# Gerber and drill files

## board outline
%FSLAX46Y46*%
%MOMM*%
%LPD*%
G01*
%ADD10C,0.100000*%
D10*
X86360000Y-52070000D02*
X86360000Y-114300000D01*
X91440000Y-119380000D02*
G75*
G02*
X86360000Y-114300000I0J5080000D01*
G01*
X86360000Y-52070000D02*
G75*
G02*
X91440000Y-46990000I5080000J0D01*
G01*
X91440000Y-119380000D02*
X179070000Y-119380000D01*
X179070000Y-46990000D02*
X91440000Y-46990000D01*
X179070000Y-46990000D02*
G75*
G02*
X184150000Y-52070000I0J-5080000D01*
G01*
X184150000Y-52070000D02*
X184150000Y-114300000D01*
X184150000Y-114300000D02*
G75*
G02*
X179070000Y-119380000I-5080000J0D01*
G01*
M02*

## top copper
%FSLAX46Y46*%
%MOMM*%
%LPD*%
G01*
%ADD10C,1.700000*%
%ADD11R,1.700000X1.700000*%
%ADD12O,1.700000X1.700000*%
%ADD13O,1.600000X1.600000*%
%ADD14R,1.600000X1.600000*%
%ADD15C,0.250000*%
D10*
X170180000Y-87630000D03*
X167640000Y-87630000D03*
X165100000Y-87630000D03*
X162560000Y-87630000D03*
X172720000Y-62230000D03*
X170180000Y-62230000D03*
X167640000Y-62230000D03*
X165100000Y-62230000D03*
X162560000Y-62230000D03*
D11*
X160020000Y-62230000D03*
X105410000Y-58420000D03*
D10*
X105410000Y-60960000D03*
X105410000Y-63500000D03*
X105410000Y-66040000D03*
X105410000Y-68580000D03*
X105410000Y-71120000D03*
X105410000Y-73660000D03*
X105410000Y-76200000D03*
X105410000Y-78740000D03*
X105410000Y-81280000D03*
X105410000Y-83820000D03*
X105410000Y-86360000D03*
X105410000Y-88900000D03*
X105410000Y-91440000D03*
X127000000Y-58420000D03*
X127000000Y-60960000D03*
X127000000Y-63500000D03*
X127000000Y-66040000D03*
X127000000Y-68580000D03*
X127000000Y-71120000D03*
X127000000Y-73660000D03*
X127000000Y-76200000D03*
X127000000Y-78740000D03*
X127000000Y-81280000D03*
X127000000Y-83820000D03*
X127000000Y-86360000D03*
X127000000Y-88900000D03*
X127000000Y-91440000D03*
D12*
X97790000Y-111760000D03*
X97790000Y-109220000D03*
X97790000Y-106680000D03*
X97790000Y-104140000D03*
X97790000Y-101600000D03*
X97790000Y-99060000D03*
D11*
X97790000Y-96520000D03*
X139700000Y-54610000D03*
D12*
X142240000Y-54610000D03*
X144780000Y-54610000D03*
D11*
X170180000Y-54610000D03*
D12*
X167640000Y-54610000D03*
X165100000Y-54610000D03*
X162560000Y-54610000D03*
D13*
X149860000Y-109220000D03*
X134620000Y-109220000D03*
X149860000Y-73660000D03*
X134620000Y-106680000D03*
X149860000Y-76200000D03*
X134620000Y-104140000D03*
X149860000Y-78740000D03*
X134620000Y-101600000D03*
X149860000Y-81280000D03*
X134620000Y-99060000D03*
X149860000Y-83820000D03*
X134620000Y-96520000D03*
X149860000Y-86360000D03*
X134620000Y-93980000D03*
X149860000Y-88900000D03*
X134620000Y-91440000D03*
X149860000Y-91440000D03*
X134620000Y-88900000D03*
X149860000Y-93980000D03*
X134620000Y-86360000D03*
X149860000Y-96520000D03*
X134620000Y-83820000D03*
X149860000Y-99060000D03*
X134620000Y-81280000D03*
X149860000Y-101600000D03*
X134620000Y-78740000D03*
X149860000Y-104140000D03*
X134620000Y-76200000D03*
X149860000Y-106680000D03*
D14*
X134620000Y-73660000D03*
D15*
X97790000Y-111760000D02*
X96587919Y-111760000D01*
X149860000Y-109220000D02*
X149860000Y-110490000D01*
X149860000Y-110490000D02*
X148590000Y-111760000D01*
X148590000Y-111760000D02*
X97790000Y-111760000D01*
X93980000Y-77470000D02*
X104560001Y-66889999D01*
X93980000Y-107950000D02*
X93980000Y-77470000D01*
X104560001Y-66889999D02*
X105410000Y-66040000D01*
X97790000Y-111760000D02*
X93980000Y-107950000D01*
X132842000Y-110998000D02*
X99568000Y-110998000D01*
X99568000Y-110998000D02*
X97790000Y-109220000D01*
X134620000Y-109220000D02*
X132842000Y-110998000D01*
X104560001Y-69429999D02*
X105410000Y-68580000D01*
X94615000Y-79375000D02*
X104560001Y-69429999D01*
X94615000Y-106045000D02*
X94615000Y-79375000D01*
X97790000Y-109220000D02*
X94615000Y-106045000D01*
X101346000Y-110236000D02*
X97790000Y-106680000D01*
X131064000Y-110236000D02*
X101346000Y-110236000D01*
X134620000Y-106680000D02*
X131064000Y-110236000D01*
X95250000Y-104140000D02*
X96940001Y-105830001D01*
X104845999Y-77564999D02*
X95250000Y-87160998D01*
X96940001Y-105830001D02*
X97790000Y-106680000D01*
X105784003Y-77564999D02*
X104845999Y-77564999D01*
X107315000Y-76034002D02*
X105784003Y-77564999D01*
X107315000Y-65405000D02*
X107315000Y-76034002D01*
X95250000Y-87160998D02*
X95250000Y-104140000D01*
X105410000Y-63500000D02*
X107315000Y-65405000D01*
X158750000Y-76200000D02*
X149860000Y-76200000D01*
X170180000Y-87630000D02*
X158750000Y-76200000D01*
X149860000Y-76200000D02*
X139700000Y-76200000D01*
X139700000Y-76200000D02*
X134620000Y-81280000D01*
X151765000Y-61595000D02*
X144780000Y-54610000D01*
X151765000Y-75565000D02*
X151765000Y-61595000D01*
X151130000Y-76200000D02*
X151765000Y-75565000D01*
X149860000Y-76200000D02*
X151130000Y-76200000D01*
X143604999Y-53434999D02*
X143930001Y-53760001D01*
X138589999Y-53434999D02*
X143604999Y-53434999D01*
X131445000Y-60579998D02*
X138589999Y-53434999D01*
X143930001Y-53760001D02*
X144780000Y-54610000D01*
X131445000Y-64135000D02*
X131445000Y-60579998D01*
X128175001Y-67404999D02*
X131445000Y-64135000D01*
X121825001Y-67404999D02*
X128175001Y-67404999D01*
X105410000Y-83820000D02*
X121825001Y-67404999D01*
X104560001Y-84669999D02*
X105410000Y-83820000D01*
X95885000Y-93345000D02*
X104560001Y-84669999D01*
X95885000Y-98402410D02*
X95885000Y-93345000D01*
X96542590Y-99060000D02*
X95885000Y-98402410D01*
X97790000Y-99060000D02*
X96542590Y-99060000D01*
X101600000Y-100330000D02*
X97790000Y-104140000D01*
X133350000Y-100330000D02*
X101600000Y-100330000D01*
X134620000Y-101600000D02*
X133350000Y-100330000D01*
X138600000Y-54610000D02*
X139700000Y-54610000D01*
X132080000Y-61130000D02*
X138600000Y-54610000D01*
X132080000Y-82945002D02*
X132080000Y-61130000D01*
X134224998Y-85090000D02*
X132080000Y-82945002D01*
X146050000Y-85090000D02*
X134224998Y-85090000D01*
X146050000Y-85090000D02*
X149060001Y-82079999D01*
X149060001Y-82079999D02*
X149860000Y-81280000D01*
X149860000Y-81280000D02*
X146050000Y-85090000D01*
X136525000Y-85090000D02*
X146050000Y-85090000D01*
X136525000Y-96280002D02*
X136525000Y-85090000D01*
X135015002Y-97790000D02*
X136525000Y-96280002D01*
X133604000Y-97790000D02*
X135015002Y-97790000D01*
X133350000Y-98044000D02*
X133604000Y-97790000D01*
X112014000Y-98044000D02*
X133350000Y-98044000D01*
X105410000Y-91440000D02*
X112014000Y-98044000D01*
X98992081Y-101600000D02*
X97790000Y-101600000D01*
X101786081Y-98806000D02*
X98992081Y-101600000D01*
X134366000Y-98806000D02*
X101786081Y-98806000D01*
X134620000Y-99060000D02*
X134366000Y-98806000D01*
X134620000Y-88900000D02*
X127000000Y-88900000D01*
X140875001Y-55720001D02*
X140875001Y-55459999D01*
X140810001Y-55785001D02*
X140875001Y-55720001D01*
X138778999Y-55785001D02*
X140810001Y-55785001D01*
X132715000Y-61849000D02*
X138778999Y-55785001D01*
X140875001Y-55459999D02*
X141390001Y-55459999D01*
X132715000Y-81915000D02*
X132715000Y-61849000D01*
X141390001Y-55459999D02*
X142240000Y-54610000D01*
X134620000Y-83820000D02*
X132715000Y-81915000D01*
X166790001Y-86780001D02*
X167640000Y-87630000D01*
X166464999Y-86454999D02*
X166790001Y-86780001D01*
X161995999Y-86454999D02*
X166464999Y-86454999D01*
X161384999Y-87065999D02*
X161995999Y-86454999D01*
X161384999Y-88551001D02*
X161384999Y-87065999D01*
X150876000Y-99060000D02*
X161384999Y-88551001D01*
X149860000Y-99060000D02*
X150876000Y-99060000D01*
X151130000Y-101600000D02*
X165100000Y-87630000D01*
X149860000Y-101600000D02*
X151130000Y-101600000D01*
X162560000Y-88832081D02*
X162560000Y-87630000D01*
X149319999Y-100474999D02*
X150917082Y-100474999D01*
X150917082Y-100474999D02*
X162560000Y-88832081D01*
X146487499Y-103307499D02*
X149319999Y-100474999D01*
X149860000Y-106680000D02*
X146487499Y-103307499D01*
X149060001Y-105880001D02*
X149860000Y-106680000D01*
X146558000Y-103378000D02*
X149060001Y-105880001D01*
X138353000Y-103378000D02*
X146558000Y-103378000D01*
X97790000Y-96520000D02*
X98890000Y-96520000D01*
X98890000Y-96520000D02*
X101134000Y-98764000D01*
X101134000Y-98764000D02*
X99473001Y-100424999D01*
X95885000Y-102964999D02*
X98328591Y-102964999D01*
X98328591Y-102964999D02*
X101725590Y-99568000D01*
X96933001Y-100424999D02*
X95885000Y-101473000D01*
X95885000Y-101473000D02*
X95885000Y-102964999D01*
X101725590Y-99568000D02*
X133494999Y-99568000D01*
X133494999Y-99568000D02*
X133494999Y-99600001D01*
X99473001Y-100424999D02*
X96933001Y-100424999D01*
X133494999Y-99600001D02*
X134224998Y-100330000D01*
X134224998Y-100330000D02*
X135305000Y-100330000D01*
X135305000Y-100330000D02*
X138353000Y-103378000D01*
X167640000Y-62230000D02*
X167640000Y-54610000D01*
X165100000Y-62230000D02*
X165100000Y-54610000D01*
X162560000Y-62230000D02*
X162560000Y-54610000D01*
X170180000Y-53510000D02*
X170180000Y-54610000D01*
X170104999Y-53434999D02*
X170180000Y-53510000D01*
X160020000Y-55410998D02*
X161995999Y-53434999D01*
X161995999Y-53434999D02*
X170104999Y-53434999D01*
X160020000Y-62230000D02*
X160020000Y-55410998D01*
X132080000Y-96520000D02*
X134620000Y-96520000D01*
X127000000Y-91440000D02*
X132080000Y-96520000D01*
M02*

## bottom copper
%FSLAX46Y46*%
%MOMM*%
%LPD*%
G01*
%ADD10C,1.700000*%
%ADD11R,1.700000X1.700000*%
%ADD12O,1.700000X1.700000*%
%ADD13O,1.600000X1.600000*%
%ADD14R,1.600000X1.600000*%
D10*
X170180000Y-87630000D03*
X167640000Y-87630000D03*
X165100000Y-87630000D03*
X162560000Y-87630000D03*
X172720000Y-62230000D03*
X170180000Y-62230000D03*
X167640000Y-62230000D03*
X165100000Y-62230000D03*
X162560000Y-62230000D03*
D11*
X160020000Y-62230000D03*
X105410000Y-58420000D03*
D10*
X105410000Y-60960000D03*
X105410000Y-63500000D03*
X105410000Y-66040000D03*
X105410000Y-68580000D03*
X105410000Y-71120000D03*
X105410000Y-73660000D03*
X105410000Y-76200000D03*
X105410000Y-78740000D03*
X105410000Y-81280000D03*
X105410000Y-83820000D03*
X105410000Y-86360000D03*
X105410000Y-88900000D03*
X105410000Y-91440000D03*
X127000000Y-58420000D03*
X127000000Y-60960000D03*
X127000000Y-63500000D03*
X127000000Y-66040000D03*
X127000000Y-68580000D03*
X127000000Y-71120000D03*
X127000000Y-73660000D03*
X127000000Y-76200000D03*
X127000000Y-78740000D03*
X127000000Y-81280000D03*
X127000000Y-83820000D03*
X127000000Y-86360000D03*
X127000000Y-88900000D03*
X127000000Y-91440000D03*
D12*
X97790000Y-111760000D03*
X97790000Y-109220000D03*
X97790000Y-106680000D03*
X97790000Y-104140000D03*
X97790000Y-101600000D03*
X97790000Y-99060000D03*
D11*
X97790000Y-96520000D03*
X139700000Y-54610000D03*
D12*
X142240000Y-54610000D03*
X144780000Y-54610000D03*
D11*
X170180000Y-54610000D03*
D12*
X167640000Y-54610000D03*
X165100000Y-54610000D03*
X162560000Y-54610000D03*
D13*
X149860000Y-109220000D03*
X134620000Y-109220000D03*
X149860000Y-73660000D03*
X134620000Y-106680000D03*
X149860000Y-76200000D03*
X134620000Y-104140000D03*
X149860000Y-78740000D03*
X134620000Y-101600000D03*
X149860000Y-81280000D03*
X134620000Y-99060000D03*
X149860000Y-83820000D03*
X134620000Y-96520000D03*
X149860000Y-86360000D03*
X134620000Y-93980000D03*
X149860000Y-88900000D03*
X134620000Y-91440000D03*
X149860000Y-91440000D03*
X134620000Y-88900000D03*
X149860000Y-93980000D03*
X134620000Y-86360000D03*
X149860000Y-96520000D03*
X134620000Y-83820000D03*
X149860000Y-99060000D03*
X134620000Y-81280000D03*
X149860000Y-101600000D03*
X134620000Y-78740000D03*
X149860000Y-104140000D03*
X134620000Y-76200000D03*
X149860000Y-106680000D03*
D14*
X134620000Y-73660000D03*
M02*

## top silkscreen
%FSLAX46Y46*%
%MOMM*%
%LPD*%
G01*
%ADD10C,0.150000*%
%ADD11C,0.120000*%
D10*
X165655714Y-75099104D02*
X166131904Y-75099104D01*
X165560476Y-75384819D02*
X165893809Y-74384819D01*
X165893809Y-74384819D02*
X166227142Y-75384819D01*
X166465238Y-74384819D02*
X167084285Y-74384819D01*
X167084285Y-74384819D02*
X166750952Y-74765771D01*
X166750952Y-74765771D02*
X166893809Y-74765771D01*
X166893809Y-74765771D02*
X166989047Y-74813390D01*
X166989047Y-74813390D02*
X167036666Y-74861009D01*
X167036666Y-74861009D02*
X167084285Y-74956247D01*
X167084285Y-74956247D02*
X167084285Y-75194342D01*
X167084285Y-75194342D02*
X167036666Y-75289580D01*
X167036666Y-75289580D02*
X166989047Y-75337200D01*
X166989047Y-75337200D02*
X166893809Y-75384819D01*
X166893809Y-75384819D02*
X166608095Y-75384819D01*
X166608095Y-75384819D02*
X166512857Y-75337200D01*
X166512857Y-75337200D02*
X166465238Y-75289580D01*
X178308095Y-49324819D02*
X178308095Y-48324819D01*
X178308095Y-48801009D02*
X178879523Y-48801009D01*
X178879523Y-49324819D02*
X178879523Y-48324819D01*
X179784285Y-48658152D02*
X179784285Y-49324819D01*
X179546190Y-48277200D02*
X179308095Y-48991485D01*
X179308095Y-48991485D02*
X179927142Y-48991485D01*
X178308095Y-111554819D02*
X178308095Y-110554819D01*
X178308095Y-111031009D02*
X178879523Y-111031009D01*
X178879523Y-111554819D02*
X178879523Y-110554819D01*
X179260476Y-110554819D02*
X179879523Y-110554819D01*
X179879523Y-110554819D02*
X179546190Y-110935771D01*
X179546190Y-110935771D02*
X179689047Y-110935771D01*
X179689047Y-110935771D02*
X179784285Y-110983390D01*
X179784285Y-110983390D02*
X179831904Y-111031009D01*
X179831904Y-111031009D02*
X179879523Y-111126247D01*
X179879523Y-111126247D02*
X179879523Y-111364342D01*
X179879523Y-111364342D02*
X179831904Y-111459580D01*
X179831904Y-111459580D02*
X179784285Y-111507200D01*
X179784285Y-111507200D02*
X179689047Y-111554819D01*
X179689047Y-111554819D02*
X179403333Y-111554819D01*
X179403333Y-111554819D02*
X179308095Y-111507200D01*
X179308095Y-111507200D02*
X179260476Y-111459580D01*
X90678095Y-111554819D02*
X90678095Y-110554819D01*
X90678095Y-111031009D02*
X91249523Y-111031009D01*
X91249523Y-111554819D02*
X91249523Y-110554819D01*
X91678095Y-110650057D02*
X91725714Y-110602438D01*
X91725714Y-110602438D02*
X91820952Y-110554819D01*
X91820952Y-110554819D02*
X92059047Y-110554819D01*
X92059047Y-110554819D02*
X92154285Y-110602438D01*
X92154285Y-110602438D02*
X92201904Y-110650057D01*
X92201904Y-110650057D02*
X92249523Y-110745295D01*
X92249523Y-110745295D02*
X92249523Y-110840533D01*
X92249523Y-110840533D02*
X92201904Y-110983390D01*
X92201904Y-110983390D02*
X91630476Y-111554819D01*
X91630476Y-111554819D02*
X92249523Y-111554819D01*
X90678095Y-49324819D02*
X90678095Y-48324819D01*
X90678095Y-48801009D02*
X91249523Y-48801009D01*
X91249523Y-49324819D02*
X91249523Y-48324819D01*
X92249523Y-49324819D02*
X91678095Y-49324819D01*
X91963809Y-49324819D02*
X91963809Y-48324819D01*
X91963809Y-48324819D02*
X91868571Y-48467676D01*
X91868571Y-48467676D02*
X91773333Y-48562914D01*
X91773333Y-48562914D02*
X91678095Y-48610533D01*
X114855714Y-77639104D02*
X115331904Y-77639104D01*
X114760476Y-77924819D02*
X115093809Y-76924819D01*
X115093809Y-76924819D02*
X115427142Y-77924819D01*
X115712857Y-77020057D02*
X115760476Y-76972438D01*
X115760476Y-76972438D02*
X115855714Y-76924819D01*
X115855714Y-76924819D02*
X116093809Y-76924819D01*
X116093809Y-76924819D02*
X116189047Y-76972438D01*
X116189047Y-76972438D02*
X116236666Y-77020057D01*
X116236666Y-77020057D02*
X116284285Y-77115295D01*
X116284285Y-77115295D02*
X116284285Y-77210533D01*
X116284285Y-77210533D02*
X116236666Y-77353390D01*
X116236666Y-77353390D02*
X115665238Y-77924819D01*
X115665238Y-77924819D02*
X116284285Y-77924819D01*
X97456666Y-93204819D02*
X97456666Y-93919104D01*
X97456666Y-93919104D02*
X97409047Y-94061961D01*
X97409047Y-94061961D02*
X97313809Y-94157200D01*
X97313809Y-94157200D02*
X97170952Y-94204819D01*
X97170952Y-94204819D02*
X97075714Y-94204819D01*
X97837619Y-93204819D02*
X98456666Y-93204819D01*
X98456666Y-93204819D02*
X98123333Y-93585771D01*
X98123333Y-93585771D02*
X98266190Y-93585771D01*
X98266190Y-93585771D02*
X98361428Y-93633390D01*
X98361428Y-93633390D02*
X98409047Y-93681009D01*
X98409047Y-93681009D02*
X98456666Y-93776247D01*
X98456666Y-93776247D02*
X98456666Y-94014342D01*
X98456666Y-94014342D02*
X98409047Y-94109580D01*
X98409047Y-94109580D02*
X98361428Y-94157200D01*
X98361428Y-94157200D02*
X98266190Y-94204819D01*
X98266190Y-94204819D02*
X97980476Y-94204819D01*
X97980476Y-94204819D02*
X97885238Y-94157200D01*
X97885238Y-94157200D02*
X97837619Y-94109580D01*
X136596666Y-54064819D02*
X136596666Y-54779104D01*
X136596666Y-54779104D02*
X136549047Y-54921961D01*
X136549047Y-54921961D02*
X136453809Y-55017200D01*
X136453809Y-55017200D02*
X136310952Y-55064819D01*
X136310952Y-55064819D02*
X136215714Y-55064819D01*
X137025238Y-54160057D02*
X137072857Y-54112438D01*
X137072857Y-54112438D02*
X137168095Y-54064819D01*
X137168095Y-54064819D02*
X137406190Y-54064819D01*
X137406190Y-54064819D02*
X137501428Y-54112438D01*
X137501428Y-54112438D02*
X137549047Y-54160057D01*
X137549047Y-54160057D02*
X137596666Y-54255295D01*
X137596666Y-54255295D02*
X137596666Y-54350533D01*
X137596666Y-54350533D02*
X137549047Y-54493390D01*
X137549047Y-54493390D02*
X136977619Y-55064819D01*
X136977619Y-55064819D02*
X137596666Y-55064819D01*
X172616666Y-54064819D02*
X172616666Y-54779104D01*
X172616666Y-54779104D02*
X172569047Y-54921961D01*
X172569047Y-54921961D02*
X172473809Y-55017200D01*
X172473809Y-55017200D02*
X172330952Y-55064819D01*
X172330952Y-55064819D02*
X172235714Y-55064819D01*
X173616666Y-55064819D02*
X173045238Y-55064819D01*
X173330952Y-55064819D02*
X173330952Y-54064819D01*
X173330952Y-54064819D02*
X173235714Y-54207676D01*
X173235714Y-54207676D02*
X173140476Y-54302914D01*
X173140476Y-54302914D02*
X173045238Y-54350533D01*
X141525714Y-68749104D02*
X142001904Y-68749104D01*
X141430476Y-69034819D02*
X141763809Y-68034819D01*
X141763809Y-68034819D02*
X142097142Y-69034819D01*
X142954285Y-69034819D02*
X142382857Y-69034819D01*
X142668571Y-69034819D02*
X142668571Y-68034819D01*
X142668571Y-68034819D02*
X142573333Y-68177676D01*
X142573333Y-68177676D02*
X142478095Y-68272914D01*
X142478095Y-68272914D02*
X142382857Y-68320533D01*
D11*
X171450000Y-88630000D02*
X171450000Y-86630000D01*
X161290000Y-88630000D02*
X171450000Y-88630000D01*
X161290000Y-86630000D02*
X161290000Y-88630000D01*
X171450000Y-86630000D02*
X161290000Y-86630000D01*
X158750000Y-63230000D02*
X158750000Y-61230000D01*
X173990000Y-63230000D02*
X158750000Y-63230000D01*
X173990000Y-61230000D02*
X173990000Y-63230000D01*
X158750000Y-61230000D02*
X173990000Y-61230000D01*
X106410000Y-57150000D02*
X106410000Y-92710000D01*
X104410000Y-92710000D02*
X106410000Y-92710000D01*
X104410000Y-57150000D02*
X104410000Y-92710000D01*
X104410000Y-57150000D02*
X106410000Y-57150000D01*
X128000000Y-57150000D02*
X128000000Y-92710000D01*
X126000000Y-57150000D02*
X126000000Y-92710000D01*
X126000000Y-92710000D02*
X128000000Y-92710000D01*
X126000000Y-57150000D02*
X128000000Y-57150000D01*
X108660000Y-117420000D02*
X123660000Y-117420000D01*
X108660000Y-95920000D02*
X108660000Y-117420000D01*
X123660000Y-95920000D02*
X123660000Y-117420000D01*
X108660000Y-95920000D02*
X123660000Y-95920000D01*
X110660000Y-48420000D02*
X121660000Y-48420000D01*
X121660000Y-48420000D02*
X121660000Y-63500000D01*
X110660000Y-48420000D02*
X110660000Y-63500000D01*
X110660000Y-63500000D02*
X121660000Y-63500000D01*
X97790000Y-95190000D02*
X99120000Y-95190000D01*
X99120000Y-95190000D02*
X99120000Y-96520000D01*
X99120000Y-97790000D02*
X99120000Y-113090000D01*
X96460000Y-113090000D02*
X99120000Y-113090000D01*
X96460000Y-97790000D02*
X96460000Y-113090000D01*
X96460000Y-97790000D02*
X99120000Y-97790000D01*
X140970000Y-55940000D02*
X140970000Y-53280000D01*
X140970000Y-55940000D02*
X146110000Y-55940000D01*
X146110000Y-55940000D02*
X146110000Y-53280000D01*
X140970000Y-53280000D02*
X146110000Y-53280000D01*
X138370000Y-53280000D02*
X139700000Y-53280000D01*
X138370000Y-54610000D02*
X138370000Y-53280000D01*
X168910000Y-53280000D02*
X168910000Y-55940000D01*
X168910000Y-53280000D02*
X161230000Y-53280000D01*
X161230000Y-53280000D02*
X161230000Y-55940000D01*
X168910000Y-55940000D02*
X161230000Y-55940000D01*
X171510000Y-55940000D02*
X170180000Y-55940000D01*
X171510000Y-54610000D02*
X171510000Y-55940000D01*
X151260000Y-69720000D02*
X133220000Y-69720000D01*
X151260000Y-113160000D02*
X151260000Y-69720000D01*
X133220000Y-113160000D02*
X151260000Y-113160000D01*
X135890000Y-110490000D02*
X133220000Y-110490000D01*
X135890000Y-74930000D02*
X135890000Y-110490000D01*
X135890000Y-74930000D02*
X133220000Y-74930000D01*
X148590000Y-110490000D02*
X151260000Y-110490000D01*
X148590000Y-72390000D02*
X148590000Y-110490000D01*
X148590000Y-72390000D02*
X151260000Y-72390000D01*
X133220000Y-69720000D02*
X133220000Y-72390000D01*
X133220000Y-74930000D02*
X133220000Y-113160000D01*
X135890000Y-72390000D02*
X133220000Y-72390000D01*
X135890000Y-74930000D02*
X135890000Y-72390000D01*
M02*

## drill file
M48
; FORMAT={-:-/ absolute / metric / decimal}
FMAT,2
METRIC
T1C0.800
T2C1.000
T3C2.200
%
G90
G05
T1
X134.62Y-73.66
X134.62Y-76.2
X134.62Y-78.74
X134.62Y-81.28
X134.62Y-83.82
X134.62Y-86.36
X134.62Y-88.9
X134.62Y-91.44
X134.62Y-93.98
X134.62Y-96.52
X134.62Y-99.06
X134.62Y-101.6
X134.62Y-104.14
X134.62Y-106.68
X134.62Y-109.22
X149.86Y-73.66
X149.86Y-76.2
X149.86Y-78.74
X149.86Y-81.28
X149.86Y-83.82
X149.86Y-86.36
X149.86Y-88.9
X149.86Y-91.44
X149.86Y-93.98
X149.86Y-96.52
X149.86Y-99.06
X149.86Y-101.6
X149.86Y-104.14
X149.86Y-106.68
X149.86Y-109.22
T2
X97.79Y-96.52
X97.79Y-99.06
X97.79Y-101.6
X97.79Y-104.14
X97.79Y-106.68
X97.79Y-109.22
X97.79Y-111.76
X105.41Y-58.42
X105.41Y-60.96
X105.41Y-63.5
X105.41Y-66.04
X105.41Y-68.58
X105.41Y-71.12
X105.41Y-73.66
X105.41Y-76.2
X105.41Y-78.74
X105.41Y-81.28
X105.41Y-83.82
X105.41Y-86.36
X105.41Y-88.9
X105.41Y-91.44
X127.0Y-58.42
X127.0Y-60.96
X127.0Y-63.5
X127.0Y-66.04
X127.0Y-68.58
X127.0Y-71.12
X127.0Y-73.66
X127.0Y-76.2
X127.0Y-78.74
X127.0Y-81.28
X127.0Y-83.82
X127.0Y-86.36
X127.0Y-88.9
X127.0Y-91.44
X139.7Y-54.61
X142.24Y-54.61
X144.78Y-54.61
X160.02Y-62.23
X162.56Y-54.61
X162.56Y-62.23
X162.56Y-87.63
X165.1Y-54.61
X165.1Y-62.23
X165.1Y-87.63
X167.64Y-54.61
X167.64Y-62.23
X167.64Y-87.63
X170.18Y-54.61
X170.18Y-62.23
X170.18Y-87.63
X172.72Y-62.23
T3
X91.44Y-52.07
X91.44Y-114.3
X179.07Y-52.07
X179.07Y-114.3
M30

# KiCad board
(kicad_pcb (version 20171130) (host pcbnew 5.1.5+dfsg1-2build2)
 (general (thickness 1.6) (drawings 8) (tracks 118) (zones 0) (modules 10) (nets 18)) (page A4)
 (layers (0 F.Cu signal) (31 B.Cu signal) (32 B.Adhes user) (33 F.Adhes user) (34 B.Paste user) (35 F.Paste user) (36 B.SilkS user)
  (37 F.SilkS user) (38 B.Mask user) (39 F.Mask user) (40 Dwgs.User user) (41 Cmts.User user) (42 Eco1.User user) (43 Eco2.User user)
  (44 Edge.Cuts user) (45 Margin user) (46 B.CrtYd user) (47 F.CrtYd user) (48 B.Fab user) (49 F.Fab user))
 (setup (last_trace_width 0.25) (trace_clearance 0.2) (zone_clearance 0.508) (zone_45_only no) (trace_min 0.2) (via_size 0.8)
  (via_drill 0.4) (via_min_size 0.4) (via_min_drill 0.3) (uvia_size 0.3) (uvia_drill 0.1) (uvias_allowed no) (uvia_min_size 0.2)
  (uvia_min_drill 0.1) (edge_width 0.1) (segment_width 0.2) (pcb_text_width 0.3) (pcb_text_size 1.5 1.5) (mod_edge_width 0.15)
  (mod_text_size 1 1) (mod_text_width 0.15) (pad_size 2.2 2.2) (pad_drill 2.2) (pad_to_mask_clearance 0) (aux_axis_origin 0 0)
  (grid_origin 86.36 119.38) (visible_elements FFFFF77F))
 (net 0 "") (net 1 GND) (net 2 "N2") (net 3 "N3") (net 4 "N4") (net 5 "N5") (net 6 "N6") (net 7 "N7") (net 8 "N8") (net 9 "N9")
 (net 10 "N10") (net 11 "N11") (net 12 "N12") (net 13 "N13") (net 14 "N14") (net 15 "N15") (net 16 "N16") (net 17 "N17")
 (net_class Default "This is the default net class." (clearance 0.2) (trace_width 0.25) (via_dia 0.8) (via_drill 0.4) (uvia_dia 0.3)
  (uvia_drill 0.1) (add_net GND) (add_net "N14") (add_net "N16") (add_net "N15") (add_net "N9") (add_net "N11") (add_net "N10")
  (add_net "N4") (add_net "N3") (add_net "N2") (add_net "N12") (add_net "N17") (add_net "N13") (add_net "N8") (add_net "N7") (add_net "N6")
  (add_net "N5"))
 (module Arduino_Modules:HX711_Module (layer F.Cu) (at 160.02 62.23)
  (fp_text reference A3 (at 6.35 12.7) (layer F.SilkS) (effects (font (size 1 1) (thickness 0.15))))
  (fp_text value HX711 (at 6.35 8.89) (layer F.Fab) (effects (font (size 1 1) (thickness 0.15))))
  (fp_line (start 11.43 26.4) (end 11.43 24.4) (layer F.SilkS) (width 0.12))
  (fp_line (start 1.27 26.4) (end 11.43 26.4) (layer F.SilkS) (width 0.12))
  (fp_line (start 1.27 24.4) (end 1.27 26.4) (layer F.SilkS) (width 0.12))
  (fp_line (start 11.43 24.4) (end 1.27 24.4) (layer F.SilkS) (width 0.12))
  (fp_line (start -1.27 1) (end -1.27 -1) (layer F.SilkS) (width 0.12))
  (fp_line (start 13.97 1) (end -1.27 1) (layer F.SilkS) (width 0.12))
  (fp_line (start 13.97 -1) (end 13.97 1) (layer F.SilkS) (width 0.12))
  (fp_line (start -1.27 -1) (end 13.97 -1) (layer F.SilkS) (width 0.12))
  (pad 10 thru_hole circle (at 10.16 25.4) (size 1.7 1.7) (drill 1) (layers *.Cu *.Mask) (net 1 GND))
  (pad 9 thru_hole circle (at 7.62 25.4) (size 1.7 1.7) (drill 1) (layers *.Cu *.Mask) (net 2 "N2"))
  (pad 8 thru_hole circle (at 5.08 25.4) (size 1.7 1.7) (drill 1) (layers *.Cu *.Mask) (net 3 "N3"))
  (pad 7 thru_hole circle (at 2.54 25.4) (size 1.7 1.7) (drill 1) (layers *.Cu *.Mask) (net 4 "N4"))
  (pad 6 thru_hole circle (at 12.7 0) (size 1.7 1.7) (drill 1) (layers *.Cu *.Mask))
  (pad 5 thru_hole circle (at 10.16 0) (size 1.7 1.7) (drill 1) (layers *.Cu *.Mask))
  (pad 4 thru_hole circle (at 7.62 0) (size 1.7 1.7) (drill 1) (layers *.Cu *.Mask) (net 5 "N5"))
  (pad 3 thru_hole circle (at 5.08 0) (size 1.7 1.7) (drill 1) (layers *.Cu *.Mask) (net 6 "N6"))
  (pad 2 thru_hole circle (at 2.54 0) (size 1.7 1.7) (drill 1) (layers *.Cu *.Mask) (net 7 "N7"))
  (pad 1 thru_hole rect (at 0 0) (size 1.7 1.7) (drill 1) (layers *.Cu *.Mask) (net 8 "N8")))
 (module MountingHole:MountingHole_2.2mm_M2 (layer F.Cu) (at 179.07 52.07)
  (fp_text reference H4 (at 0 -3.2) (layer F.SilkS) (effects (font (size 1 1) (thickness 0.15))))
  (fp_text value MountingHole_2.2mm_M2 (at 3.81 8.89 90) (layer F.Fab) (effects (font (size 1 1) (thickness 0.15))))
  (pad 1 np_thru_hole circle (at 0 0) (size 2.2 2.2) (drill 2.2) (layers *.Cu *.Mask)))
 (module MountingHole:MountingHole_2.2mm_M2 (layer F.Cu) (at 179.07 114.3)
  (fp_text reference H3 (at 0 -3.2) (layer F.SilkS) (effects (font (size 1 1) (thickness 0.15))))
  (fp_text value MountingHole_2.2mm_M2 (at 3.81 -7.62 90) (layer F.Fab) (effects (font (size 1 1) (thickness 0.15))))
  (pad 1 np_thru_hole circle (at 0 0) (size 2.2 2.2) (drill 2.2) (layers *.Cu *.Mask)))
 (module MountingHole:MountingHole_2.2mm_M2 (layer F.Cu) (at 91.44 114.3)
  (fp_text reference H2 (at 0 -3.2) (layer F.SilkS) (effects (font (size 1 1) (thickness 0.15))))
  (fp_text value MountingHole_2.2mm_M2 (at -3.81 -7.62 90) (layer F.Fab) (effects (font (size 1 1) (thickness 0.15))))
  (pad 1 np_thru_hole circle (at 0 0) (size 2.2 2.2) (drill 2.2) (layers *.Cu *.Mask)))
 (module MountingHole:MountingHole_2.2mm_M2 (layer F.Cu) (at 91.44 52.07)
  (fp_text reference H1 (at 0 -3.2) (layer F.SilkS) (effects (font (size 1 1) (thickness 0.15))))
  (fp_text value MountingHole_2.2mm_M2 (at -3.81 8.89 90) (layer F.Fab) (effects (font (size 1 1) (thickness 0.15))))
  (pad "" np_thru_hole circle (at 0 0) (size 2.2 2.2) (drill 2.2) (layers *.Cu *.Mask)))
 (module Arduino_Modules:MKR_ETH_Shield (layer F.Cu) (at 105.41 58.42)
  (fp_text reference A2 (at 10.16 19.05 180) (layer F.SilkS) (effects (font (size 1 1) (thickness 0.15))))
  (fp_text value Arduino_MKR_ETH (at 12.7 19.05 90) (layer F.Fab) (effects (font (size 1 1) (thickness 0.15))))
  (fp_line (start 1 -1.27) (end 1 34.29) (layer F.SilkS) (width 0.12))
  (fp_line (start -1 34.29) (end 1 34.29) (layer F.SilkS) (width 0.12))
  (fp_line (start -1 -1.27) (end -1 34.29) (layer F.SilkS) (width 0.12))
  (fp_line (start -1 -1.27) (end 1 -1.27) (layer F.SilkS) (width 0.12))
  (fp_line (start 22.59 -1.27) (end 22.59 34.29) (layer F.SilkS) (width 0.12))
  (fp_line (start 20.59 -1.27) (end 20.59 34.29) (layer F.SilkS) (width 0.12))
  (fp_line (start 20.59 34.29) (end 22.59 34.29) (layer F.SilkS) (width 0.12))
  (fp_line (start 20.59 -1.27) (end 22.59 -1.27) (layer F.SilkS) (width 0.12))
  (fp_line (start 3.25 59) (end 18.25 59) (layer F.SilkS) (width 0.12))
  (fp_line (start 3.25 37.5) (end 3.25 59) (layer F.SilkS) (width 0.12))
  (fp_line (start 18.25 37.5) (end 18.25 59) (layer F.SilkS) (width 0.12))
  (fp_line (start 3.25 37.5) (end 18.25 37.5) (layer F.SilkS) (width 0.12))
  (fp_line (start 5.25 -10) (end 16.25 -10) (layer F.SilkS) (width 0.12))
  (fp_line (start 16.25 -10) (end 16.25 5.08) (layer F.SilkS) (width 0.12))
  (fp_line (start 5.25 -10) (end 5.25 5.08) (layer F.SilkS) (width 0.12))
  (fp_line (start 5.25 5.08) (end 16.25 5.08) (layer F.SilkS) (width 0.12))
  (pad 1 thru_hole rect (at 0 0) (size 1.7 1.7) (drill 1) (layers *.Cu *.Mask))
  (pad 2 thru_hole circle (at 0 2.54) (size 1.7 1.7) (drill 1) (layers *.Cu *.Mask))
  (pad 3 thru_hole circle (at 0 5.08) (size 1.7 1.7) (drill 1) (layers *.Cu *.Mask) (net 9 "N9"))
  (pad 4 thru_hole circle (at 0 7.62) (size 1.7 1.7) (drill 1) (layers *.Cu *.Mask) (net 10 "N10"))
  (pad 5 thru_hole circle (at 0 10.16) (size 1.7 1.7) (drill 1) (layers *.Cu *.Mask) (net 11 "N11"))
  (pad 6 thru_hole circle (at 0 12.7) (size 1.7 1.7) (drill 1) (layers *.Cu *.Mask))
  (pad 7 thru_hole circle (at 0 15.24) (size 1.7 1.7) (drill 1) (layers *.Cu *.Mask))
  (pad 8 thru_hole circle (at 0 17.78) (size 1.7 1.7) (drill 1) (layers *.Cu *.Mask))
  (pad 9 thru_hole circle (at 0 20.32) (size 1.7 1.7) (drill 1) (layers *.Cu *.Mask))
  (pad 10 thru_hole circle (at 0 22.86) (size 1.7 1.7) (drill 1) (layers *.Cu *.Mask))
  (pad 11 thru_hole circle (at 0 25.4) (size 1.7 1.7) (drill 1) (layers *.Cu *.Mask) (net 1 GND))
  (pad 12 thru_hole circle (at 0 27.94) (size 1.7 1.7) (drill 1) (layers *.Cu *.Mask))
  (pad 13 thru_hole circle (at 0 30.48) (size 1.7 1.7) (drill 1) (layers *.Cu *.Mask))
  (pad 14 thru_hole circle (at 0 33.02) (size 1.7 1.7) (drill 1) (layers *.Cu *.Mask) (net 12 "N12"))
  (pad 15 thru_hole circle (at 21.59 0) (size 1.7 1.7) (drill 1) (layers *.Cu *.Mask))
  (pad 16 thru_hole circle (at 21.59 2.54) (size 1.7 1.7) (drill 1) (layers *.Cu *.Mask))
  (pad 17 thru_hole circle (at 21.59 5.08) (size 1.7 1.7) (drill 1) (layers *.Cu *.Mask))
  (pad 18 thru_hole circle (at 21.59 7.62) (size 1.7 1.7) (drill 1) (layers *.Cu *.Mask))
  (pad 19 thru_hole circle (at 21.59 10.16) (size 1.7 1.7) (drill 1) (layers *.Cu *.Mask))
  (pad 20 thru_hole circle (at 21.59 12.7) (size 1.7 1.7) (drill 1) (layers *.Cu *.Mask))
  (pad 21 thru_hole circle (at 21.59 15.24) (size 1.7 1.7) (drill 1) (layers *.Cu *.Mask))
  (pad 22 thru_hole circle (at 21.59 17.78) (size 1.7 1.7) (drill 1) (layers *.Cu *.Mask))
  (pad 23 thru_hole circle (at 21.59 20.32) (size 1.7 1.7) (drill 1) (layers *.Cu *.Mask))
  (pad 24 thru_hole circle (at 21.59 22.86) (size 1.7 1.7) (drill 1) (layers *.Cu *.Mask))
  (pad 25 thru_hole circle (at 21.59 25.4) (size 1.7 1.7) (drill 1) (layers *.Cu *.Mask))
  (pad 26 thru_hole circle (at 21.59 27.94) (size 1.7 1.7) (drill 1) (layers *.Cu *.Mask))
  (pad 27 thru_hole circle (at 21.59 30.48) (size 1.7 1.7) (drill 1) (layers *.Cu *.Mask) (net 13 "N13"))
  (pad 28 thru_hole circle (at 21.59 33.02) (size 1.7 1.7) (drill 1) (layers *.Cu *.Mask) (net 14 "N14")))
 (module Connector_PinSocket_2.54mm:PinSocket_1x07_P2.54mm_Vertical (layer F.Cu) (at 97.79 96.52)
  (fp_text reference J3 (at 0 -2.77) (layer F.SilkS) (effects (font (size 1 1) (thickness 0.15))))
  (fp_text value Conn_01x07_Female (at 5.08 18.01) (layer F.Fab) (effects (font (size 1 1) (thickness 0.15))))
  (fp_line (start 0 -1.33) (end 1.33 -1.33) (layer F.SilkS) (width 0.12))
  (fp_line (start 1.33 -1.33) (end 1.33 0) (layer F.SilkS) (width 0.12))
  (fp_line (start 1.33 1.27) (end 1.33 16.57) (layer F.SilkS) (width 0.12))
  (fp_line (start -1.33 16.57) (end 1.33 16.57) (layer F.SilkS) (width 0.12))
  (fp_line (start -1.33 1.27) (end -1.33 16.57) (layer F.SilkS) (width 0.12))
  (fp_line (start -1.33 1.27) (end 1.33 1.27) (layer F.SilkS) (width 0.12))
  (pad 7 thru_hole oval (at 0 15.24) (size 1.7 1.7) (drill 1) (layers *.Cu *.Mask) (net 10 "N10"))
  (pad 6 thru_hole oval (at 0 12.7) (size 1.7 1.7) (drill 1) (layers *.Cu *.Mask) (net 11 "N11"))
  (pad 5 thru_hole oval (at 0 10.16) (size 1.7 1.7) (drill 1) (layers *.Cu *.Mask) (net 9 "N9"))
  (pad 4 thru_hole oval (at 0 7.62) (size 1.7 1.7) (drill 1) (layers *.Cu *.Mask) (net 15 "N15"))
  (pad 3 thru_hole oval (at 0 5.08) (size 1.7 1.7) (drill 1) (layers *.Cu *.Mask) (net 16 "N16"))
  (pad 2 thru_hole oval (at 0 2.54) (size 1.7 1.7) (drill 1) (layers *.Cu *.Mask) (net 1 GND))
  (pad 1 thru_hole rect (at 0 0) (size 1.7 1.7) (drill 1) (layers *.Cu *.Mask) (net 4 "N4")))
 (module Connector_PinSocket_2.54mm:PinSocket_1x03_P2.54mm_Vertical (layer F.Cu) (at 139.7 54.61 90)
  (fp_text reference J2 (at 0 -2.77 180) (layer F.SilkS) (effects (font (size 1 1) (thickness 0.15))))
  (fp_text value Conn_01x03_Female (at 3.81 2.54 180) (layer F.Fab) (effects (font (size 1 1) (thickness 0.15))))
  (fp_line (start -1.33 1.27) (end 1.33 1.27) (layer F.SilkS) (width 0.12))
  (fp_line (start -1.33 1.27) (end -1.33 6.41) (layer F.SilkS) (width 0.12))
  (fp_line (start -1.33 6.41) (end 1.33 6.41) (layer F.SilkS) (width 0.12))
  (fp_line (start 1.33 1.27) (end 1.33 6.41) (layer F.SilkS) (width 0.12))
  (fp_line (start 1.33 -1.33) (end 1.33 0) (layer F.SilkS) (width 0.12))
  (fp_line (start 0 -1.33) (end 1.33 -1.33) (layer F.SilkS) (width 0.12))
  (pad 1 thru_hole rect (at 0 0 90) (size 1.7 1.7) (drill 1) (layers *.Cu *.Mask) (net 12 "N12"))
  (pad 2 thru_hole oval (at 0 2.54 90) (size 1.7 1.7) (drill 1) (layers *.Cu *.Mask) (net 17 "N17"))
  (pad 3 thru_hole oval (at 0 5.08 90) (size 1.7 1.7) (drill 1) (layers *.Cu *.Mask) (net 1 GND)))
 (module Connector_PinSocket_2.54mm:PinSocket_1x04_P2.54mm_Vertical (layer F.Cu) (at 170.18 54.61 270)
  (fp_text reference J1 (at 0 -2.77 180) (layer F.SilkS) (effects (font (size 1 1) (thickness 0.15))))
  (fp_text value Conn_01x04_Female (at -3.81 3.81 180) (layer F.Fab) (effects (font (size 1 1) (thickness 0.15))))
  (fp_line (start -1.33 1.27) (end 1.33 1.27) (layer F.SilkS) (width 0.12))
  (fp_line (start -1.33 1.27) (end -1.33 8.95) (layer F.SilkS) (width 0.12))
  (fp_line (start -1.33 8.95) (end 1.33 8.95) (layer F.SilkS) (width 0.12))
  (fp_line (start 1.33 1.27) (end 1.33 8.95) (layer F.SilkS) (width 0.12))
  (fp_line (start 1.33 -1.33) (end 1.33 0) (layer F.SilkS) (width 0.12))
  (fp_line (start 0 -1.33) (end 1.33 -1.33) (layer F.SilkS) (width 0.12))
  (pad 1 thru_hole rect (at 0 0 270) (size 1.7 1.7) (drill 1) (layers *.Cu *.Mask) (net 8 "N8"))
  (pad 2 thru_hole oval (at 0 2.54 270) (size 1.7 1.7) (drill 1) (layers *.Cu *.Mask) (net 5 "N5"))
  (pad 3 thru_hole oval (at 0 5.08 270) (size 1.7 1.7) (drill 1) (layers *.Cu *.Mask) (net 6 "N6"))
  (pad 4 thru_hole oval (at 0 7.62 270) (size 1.7 1.7) (drill 1) (layers *.Cu *.Mask) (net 7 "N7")))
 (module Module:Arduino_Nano (layer F.Cu) (at 134.62 73.66)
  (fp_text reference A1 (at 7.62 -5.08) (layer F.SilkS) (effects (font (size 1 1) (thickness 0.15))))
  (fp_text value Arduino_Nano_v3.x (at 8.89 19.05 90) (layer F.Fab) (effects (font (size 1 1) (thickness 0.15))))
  (fp_line (start 16.64 -3.94) (end -1.4 -3.94) (layer F.SilkS) (width 0.12))
  (fp_line (start 16.64 39.5) (end 16.64 -3.94) (layer F.SilkS) (width 0.12))
  (fp_line (start -1.4 39.5) (end 16.64 39.5) (layer F.SilkS) (width 0.12))
  (fp_line (start 1.27 36.83) (end -1.4 36.83) (layer F.SilkS) (width 0.12))
  (fp_line (start 1.27 1.27) (end 1.27 36.83) (layer F.SilkS) (width 0.12))
  (fp_line (start 1.27 1.27) (end -1.4 1.27) (layer F.SilkS) (width 0.12))
  (fp_line (start 13.97 36.83) (end 16.64 36.83) (layer F.SilkS) (width 0.12))
  (fp_line (start 13.97 -1.27) (end 13.97 36.83) (layer F.SilkS) (width 0.12))
  (fp_line (start 13.97 -1.27) (end 16.64 -1.27) (layer F.SilkS) (width 0.12))
  (fp_line (start -1.4 -3.94) (end -1.4 -1.27) (layer F.SilkS) (width 0.12))
  (fp_line (start -1.4 1.27) (end -1.4 39.5) (layer F.SilkS) (width 0.12))
  (fp_line (start 1.27 -1.27) (end -1.4 -1.27) (layer F.SilkS) (width 0.12))
  (fp_line (start 1.27 1.27) (end 1.27 -1.27) (layer F.SilkS) (width 0.12))
  (pad 16 thru_hole oval (at 15.24 35.56) (size 1.6 1.6) (drill 0.8) (layers *.Cu *.Mask) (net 10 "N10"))
  (pad 15 thru_hole oval (at 0 35.56) (size 1.6 1.6) (drill 0.8) (layers *.Cu *.Mask) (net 11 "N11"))
  (pad 30 thru_hole oval (at 15.24 0) (size 1.6 1.6) (drill 0.8) (layers *.Cu *.Mask))
  (pad 14 thru_hole oval (at 0 33.02) (size 1.6 1.6) (drill 0.8) (layers *.Cu *.Mask) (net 9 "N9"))
  (pad 29 thru_hole oval (at 15.24 2.54) (size 1.6 1.6) (drill 0.8) (layers *.Cu *.Mask) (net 1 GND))
  (pad 13 thru_hole oval (at 0 30.48) (size 1.6 1.6) (drill 0.8) (layers *.Cu *.Mask))
  (pad 28 thru_hole oval (at 15.24 5.08) (size 1.6 1.6) (drill 0.8) (layers *.Cu *.Mask))
  (pad 12 thru_hole oval (at 0 27.94) (size 1.6 1.6) (drill 0.8) (layers *.Cu *.Mask) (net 15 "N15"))
  (pad 27 thru_hole oval (at 15.24 7.62) (size 1.6 1.6) (drill 0.8) (layers *.Cu *.Mask) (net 12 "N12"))
  (pad 11 thru_hole oval (at 0 25.4) (size 1.6 1.6) (drill 0.8) (layers *.Cu *.Mask) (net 16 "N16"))
  (pad 26 thru_hole oval (at 15.24 10.16) (size 1.6 1.6) (drill 0.8) (layers *.Cu *.Mask))
  (pad 10 thru_hole oval (at 0 22.86) (size 1.6 1.6) (drill 0.8) (layers *.Cu *.Mask) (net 14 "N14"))
  (pad 25 thru_hole oval (at 15.24 12.7) (size 1.6 1.6) (drill 0.8) (layers *.Cu *.Mask))
  (pad 9 thru_hole oval (at 0 20.32) (size 1.6 1.6) (drill 0.8) (layers *.Cu *.Mask))
  (pad 24 thru_hole oval (at 15.24 15.24) (size 1.6 1.6) (drill 0.8) (layers *.Cu *.Mask))
  (pad 8 thru_hole oval (at 0 17.78) (size 1.6 1.6) (drill 0.8) (layers *.Cu *.Mask))
  (pad 23 thru_hole oval (at 15.24 17.78) (size 1.6 1.6) (drill 0.8) (layers *.Cu *.Mask))
  (pad 7 thru_hole oval (at 0 15.24) (size 1.6 1.6) (drill 0.8) (layers *.Cu *.Mask) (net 13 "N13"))
  (pad 22 thru_hole oval (at 15.24 20.32) (size 1.6 1.6) (drill 0.8) (layers *.Cu *.Mask))
  (pad 6 thru_hole oval (at 0 12.7) (size 1.6 1.6) (drill 0.8) (layers *.Cu *.Mask))
  (pad 21 thru_hole oval (at 15.24 22.86) (size 1.6 1.6) (drill 0.8) (layers *.Cu *.Mask))
  (pad 5 thru_hole oval (at 0 10.16) (size 1.6 1.6) (drill 0.8) (layers *.Cu *.Mask) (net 17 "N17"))
  (pad 20 thru_hole oval (at 15.24 25.4) (size 1.6 1.6) (drill 0.8) (layers *.Cu *.Mask) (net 2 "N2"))
  (pad 4 thru_hole oval (at 0 7.62) (size 1.6 1.6) (drill 0.8) (layers *.Cu *.Mask) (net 1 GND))
  (pad 19 thru_hole oval (at 15.24 27.94) (size 1.6 1.6) (drill 0.8) (layers *.Cu *.Mask) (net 3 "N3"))
  (pad 3 thru_hole oval (at 0 5.08) (size 1.6 1.6) (drill 0.8) (layers *.Cu *.Mask))
  (pad 18 thru_hole oval (at 15.24 30.48) (size 1.6 1.6) (drill 0.8) (layers *.Cu *.Mask))
  (pad 2 thru_hole oval (at 0 2.54) (size 1.6 1.6) (drill 0.8) (layers *.Cu *.Mask))
  (pad 17 thru_hole oval (at 15.24 33.02) (size 1.6 1.6) (drill 0.8) (layers *.Cu *.Mask) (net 4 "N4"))
  (pad 1 thru_hole rect (at 0 0) (size 1.6 1.6) (drill 0.8) (layers *.Cu *.Mask)))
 (gr_line (start 86.36 52.07) (end 86.36 114.3) (layer Edge.Cuts) (width 0.1))
 (gr_arc (start 91.44 114.3) (end 86.36 114.3) (angle -90) (layer Edge.Cuts) (width 0.1))
 (gr_arc (start 91.44 52.07) (end 91.44 46.99) (angle -90) (layer Edge.Cuts) (width 0.1))
 (gr_line (start 91.44 119.38) (end 179.07 119.38) (layer Edge.Cuts) (width 0.1))
 (gr_line (start 179.07 46.99) (end 91.44 46.99) (layer Edge.Cuts) (width 0.1))
 (gr_arc (start 179.07 52.07) (end 184.15 52.07) (angle -90) (layer Edge.Cuts) (width 0.1))
 (gr_line (start 184.15 52.07) (end 184.15 114.3) (layer Edge.Cuts) (width 0.1))
 (gr_arc (start 179.07 114.3) (end 179.07 119.38) (angle -90) (layer Edge.Cuts) (width 0.1))
 (segment (start 97.79 111.76) (end 96.587919 111.76) (width 0.25) (layer F.Cu) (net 10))
 (segment (start 149.86 109.22) (end 149.86 110.49) (width 0.25) (layer F.Cu) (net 10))
 (segment (start 149.86 110.49) (end 148.59 111.76) (width 0.25) (layer F.Cu) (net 10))
 (segment (start 148.59 111.76) (end 97.79 111.76) (width 0.25) (layer F.Cu) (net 10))
 (segment (start 93.98 77.47) (end 104.560001 66.889999) (width 0.25) (layer F.Cu) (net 10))
 (segment (start 93.98 107.95) (end 93.98 77.47) (width 0.25) (layer F.Cu) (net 10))
 (segment (start 104.560001 66.889999) (end 105.41 66.04) (width 0.25) (layer F.Cu) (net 10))
 (segment (start 97.79 111.76) (end 93.98 107.95) (width 0.25) (layer F.Cu) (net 10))
 (segment (start 132.842 110.998) (end 99.568 110.998) (width 0.25) (layer F.Cu) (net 11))
 (segment (start 99.568 110.998) (end 97.79 109.22) (width 0.25) (layer F.Cu) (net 11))
 (segment (start 134.62 109.22) (end 132.842 110.998) (width 0.25) (layer F.Cu) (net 11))
 (segment (start 104.560001 69.429999) (end 105.41 68.58) (width 0.25) (layer F.Cu) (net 11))
 (segment (start 94.615 79.375) (end 104.560001 69.429999) (width 0.25) (layer F.Cu) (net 11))
 (segment (start 94.615 106.045) (end 94.615 79.375) (width 0.25) (layer F.Cu) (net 11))
 (segment (start 97.79 109.22) (end 94.615 106.045) (width 0.25) (layer F.Cu) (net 11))
 (segment (start 101.346 110.236) (end 97.79 106.68) (width 0.25) (layer F.Cu) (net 9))
 (segment (start 131.064 110.236) (end 101.346 110.236) (width 0.25) (layer F.Cu) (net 9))
 (segment (start 134.62 106.68) (end 131.064 110.236) (width 0.25) (layer F.Cu) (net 9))
 (segment (start 95.25 104.14) (end 96.940001 105.830001) (width 0.25) (layer F.Cu) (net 9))
 (segment (start 104.845999 77.564999) (end 95.25 87.160998) (width 0.25) (layer F.Cu) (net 9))
 (segment (start 96.940001 105.830001) (end 97.79 106.68) (width 0.25) (layer F.Cu) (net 9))
 (segment (start 105.784003 77.564999) (end 104.845999 77.564999) (width 0.25) (layer F.Cu) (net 9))
 (segment (start 107.315 76.034002) (end 105.784003 77.564999) (width 0.25) (layer F.Cu) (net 9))
 (segment (start 107.315 65.405) (end 107.315 76.034002) (width 0.25) (layer F.Cu) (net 9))
 (segment (start 95.25 87.160998) (end 95.25 104.14) (width 0.25) (layer F.Cu) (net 9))
 (segment (start 105.41 63.5) (end 107.315 65.405) (width 0.25) (layer F.Cu) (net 9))
 (segment (start 158.75 76.2) (end 149.86 76.2) (width 0.25) (layer F.Cu) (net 1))
 (segment (start 170.18 87.63) (end 158.75 76.2) (width 0.25) (layer F.Cu) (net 1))
 (segment (start 149.86 76.2) (end 139.7 76.2) (width 0.25) (layer F.Cu) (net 1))
 (segment (start 139.7 76.2) (end 134.62 81.28) (width 0.25) (layer F.Cu) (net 1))
 (segment (start 151.765 61.595) (end 144.78 54.61) (width 0.25) (layer F.Cu) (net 1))
 (segment (start 151.765 75.565) (end 151.765 61.595) (width 0.25) (layer F.Cu) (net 1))
 (segment (start 151.13 76.2) (end 151.765 75.565) (width 0.25) (layer F.Cu) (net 1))
 (segment (start 149.86 76.2) (end 151.13 76.2) (width 0.25) (layer F.Cu) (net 1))
 (segment (start 143.604999 53.434999) (end 143.930001 53.760001) (width 0.25) (layer F.Cu) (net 1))
 (segment (start 138.589999 53.434999) (end 143.604999 53.434999) (width 0.25) (layer F.Cu) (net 1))
 (segment (start 131.445 60.579998) (end 138.589999 53.434999) (width 0.25) (layer F.Cu) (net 1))
 (segment (start 143.930001 53.760001) (end 144.78 54.61) (width 0.25) (layer F.Cu) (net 1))
 (segment (start 131.445 64.135) (end 131.445 60.579998) (width 0.25) (layer F.Cu) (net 1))
 (segment (start 128.175001 67.404999) (end 131.445 64.135) (width 0.25) (layer F.Cu) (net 1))
 (segment (start 121.825001 67.404999) (end 128.175001 67.404999) (width 0.25) (layer F.Cu) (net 1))
 (segment (start 105.41 83.82) (end 121.825001 67.404999) (width 0.25) (layer F.Cu) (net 1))
 (segment (start 104.560001 84.669999) (end 105.41 83.82) (width 0.25) (layer F.Cu) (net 1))
 (segment (start 95.885 93.345) (end 104.560001 84.669999) (width 0.25) (layer F.Cu) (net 1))
 (segment (start 95.885 98.40241) (end 95.885 93.345) (width 0.25) (layer F.Cu) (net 1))
 (segment (start 96.54259 99.06) (end 95.885 98.40241) (width 0.25) (layer F.Cu) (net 1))
 (segment (start 97.79 99.06) (end 96.54259 99.06) (width 0.25) (layer F.Cu) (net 1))
 (segment (start 101.6 100.33) (end 97.79 104.14) (width 0.25) (layer F.Cu) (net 15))
 (segment (start 133.35 100.33) (end 101.6 100.33) (width 0.25) (layer F.Cu) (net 15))
 (segment (start 134.62 101.6) (end 133.35 100.33) (width 0.25) (layer F.Cu) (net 15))
 (segment (start 138.6 54.61) (end 139.7 54.61) (width 0.25) (layer F.Cu) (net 12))
 (segment (start 132.08 61.13) (end 138.6 54.61) (width 0.25) (layer F.Cu) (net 12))
 (segment (start 132.08 82.945002) (end 132.08 61.13) (width 0.25) (layer F.Cu) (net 12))
 (segment (start 134.224998 85.09) (end 132.08 82.945002) (width 0.25) (layer F.Cu) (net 12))
 (segment (start 146.05 85.09) (end 134.224998 85.09) (width 0.25) (layer F.Cu) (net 12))
 (segment (start 146.05 85.09) (end 149.060001 82.079999) (width 0.25) (layer F.Cu) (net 12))
 (segment (start 149.060001 82.079999) (end 149.86 81.28) (width 0.25) (layer F.Cu) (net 12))
 (segment (start 149.86 81.28) (end 146.05 85.09) (width 0.25) (layer F.Cu) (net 12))
 (segment (start 136.525 85.09) (end 146.05 85.09) (width 0.25) (layer F.Cu) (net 12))
 (segment (start 136.525 96.280002) (end 136.525 85.09) (width 0.25) (layer F.Cu) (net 12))
 (segment (start 135.015002 97.79) (end 136.525 96.280002) (width 0.25) (layer F.Cu) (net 12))
 (segment (start 133.604 97.79) (end 135.015002 97.79) (width 0.25) (layer F.Cu) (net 12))
 (segment (start 133.35 98.044) (end 133.604 97.79) (width 0.25) (layer F.Cu) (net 12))
 (segment (start 112.014 98.044) (end 133.35 98.044) (width 0.25) (layer F.Cu) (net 12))
 (segment (start 105.41 91.44) (end 112.014 98.044) (width 0.25) (layer F.Cu) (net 12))
 (segment (start 98.992081 101.6) (end 97.79 101.6) (width 0.25) (layer F.Cu) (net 16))
 (segment (start 101.786081 98.806) (end 98.992081 101.6) (width 0.25) (layer F.Cu) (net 16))
 (segment (start 134.366 98.806) (end 101.786081 98.806) (width 0.25) (layer F.Cu) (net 16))
 (segment (start 134.62 99.06) (end 134.366 98.806) (width 0.25) (layer F.Cu) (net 16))
 (segment (start 134.62 88.9) (end 127 88.9) (width 0.25) (layer F.Cu) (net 13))
 (segment (start 140.875001 55.720001) (end 140.875001 55.459999) (width 0.25) (layer F.Cu) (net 17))
 (segment (start 140.810001 55.785001) (end 140.875001 55.720001) (width 0.25) (layer F.Cu) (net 17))
 (segment (start 138.778999 55.785001) (end 140.810001 55.785001) (width 0.25) (layer F.Cu) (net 17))
 (segment (start 132.715 61.849) (end 138.778999 55.785001) (width 0.25) (layer F.Cu) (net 17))
 (segment (start 140.875001 55.459999) (end 141.390001 55.459999) (width 0.25) (layer F.Cu) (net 17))
 (segment (start 132.715 81.915) (end 132.715 61.849) (width 0.25) (layer F.Cu) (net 17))
 (segment (start 141.390001 55.459999) (end 142.24 54.61) (width 0.25) (layer F.Cu) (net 17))
 (segment (start 134.62 83.82) (end 132.715 81.915) (width 0.25) (layer F.Cu) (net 17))
 (segment (start 166.790001 86.780001) (end 167.64 87.63) (width 0.25) (layer F.Cu) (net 2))
 (segment (start 166.464999 86.454999) (end 166.790001 86.780001) (width 0.25) (layer F.Cu) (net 2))
 (segment (start 161.995999 86.454999) (end 166.464999 86.454999) (width 0.25) (layer F.Cu) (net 2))
 (segment (start 161.384999 87.065999) (end 161.995999 86.454999) (width 0.25) (layer F.Cu) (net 2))
 (segment (start 161.384999 88.551001) (end 161.384999 87.065999) (width 0.25) (layer F.Cu) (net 2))
 (segment (start 150.876 99.06) (end 161.384999 88.551001) (width 0.25) (layer F.Cu) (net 2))
 (segment (start 149.86 99.06) (end 150.876 99.06) (width 0.25) (layer F.Cu) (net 2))
 (segment (start 151.13 101.6) (end 165.1 87.63) (width 0.25) (layer F.Cu) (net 3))
 (segment (start 149.86 101.6) (end 151.13 101.6) (width 0.25) (layer F.Cu) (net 3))
 (segment (start 162.56 88.832081) (end 162.56 87.63) (width 0.25) (layer F.Cu) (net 4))
 (segment (start 149.319999 100.474999) (end 150.917082 100.474999) (width 0.25) (layer F.Cu) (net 4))
 (segment (start 150.917082 100.474999) (end 162.56 88.832081) (width 0.25) (layer F.Cu) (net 4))
 (segment (start 146.487499 103.307499) (end 149.319999 100.474999) (width 0.25) (layer F.Cu) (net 4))
 (segment (start 149.86 106.68) (end 146.487499 103.307499) (width 0.25) (layer F.Cu) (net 4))
 (segment (start 149.060001 105.880001) (end 149.86 106.68) (width 0.25) (layer F.Cu) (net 4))
 (segment (start 146.558 103.378) (end 149.060001 105.880001) (width 0.25) (layer F.Cu) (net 4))
 (segment (start 138.353 103.378) (end 146.558 103.378) (width 0.25) (layer F.Cu) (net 4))
 (segment (start 97.79 96.52) (end 98.89 96.52) (width 0.25) (layer F.Cu) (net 4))
 (segment (start 98.89 96.52) (end 101.134 98.764) (width 0.25) (layer F.Cu) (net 4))
 (segment (start 101.134 98.764) (end 99.473001 100.424999) (width 0.25) (layer F.Cu) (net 4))
 (segment (start 95.885 102.964999) (end 98.328591 102.964999) (width 0.25) (layer F.Cu) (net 4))
 (segment (start 98.328591 102.964999) (end 101.72559 99.568) (width 0.25) (layer F.Cu) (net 4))
 (segment (start 96.933001 100.424999) (end 95.885 101.473) (width 0.25) (layer F.Cu) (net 4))
 (segment (start 95.885 101.473) (end 95.885 102.964999) (width 0.25) (layer F.Cu) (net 4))
 (segment (start 101.72559 99.568) (end 133.494999 99.568) (width 0.25) (layer F.Cu) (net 4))
 (segment (start 133.494999 99.568) (end 133.494999 99.600001) (width 0.25) (layer F.Cu) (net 4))
 (segment (start 99.473001 100.424999) (end 96.933001 100.424999) (width 0.25) (layer F.Cu) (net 4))
 (segment (start 133.494999 99.600001) (end 134.224998 100.33) (width 0.25) (layer F.Cu) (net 4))
 (segment (start 134.224998 100.33) (end 135.305 100.33) (width 0.25) (layer F.Cu) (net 4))
 (segment (start 135.305 100.33) (end 138.353 103.378) (width 0.25) (layer F.Cu) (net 4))
 (segment (start 167.64 62.23) (end 167.64 54.61) (width 0.25) (layer F.Cu) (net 5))
 (segment (start 165.1 62.23) (end 165.1 54.61) (width 0.25) (layer F.Cu) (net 6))
 (segment (start 162.56 62.23) (end 162.56 54.61) (width 0.25) (layer F.Cu) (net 7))
 (segment (start 170.18 53.51) (end 170.18 54.61) (width 0.25) (layer F.Cu) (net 8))
 (segment (start 170.104999 53.434999) (end 170.18 53.51) (width 0.25) (layer F.Cu) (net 8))
 (segment (start 160.02 55.410998) (end 161.995999 53.434999) (width 0.25) (layer F.Cu) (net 8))
 (segment (start 161.995999 53.434999) (end 170.104999 53.434999) (width 0.25) (layer F.Cu) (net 8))
 (segment (start 160.02 62.23) (end 160.02 55.410998) (width 0.25) (layer F.Cu) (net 8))
 (segment (start 132.08 96.52) (end 134.62 96.52) (width 0.25) (layer F.Cu) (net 14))
 (segment (start 127 91.44) (end 132.08 96.52) (width 0.25) (layer F.Cu) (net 14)))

